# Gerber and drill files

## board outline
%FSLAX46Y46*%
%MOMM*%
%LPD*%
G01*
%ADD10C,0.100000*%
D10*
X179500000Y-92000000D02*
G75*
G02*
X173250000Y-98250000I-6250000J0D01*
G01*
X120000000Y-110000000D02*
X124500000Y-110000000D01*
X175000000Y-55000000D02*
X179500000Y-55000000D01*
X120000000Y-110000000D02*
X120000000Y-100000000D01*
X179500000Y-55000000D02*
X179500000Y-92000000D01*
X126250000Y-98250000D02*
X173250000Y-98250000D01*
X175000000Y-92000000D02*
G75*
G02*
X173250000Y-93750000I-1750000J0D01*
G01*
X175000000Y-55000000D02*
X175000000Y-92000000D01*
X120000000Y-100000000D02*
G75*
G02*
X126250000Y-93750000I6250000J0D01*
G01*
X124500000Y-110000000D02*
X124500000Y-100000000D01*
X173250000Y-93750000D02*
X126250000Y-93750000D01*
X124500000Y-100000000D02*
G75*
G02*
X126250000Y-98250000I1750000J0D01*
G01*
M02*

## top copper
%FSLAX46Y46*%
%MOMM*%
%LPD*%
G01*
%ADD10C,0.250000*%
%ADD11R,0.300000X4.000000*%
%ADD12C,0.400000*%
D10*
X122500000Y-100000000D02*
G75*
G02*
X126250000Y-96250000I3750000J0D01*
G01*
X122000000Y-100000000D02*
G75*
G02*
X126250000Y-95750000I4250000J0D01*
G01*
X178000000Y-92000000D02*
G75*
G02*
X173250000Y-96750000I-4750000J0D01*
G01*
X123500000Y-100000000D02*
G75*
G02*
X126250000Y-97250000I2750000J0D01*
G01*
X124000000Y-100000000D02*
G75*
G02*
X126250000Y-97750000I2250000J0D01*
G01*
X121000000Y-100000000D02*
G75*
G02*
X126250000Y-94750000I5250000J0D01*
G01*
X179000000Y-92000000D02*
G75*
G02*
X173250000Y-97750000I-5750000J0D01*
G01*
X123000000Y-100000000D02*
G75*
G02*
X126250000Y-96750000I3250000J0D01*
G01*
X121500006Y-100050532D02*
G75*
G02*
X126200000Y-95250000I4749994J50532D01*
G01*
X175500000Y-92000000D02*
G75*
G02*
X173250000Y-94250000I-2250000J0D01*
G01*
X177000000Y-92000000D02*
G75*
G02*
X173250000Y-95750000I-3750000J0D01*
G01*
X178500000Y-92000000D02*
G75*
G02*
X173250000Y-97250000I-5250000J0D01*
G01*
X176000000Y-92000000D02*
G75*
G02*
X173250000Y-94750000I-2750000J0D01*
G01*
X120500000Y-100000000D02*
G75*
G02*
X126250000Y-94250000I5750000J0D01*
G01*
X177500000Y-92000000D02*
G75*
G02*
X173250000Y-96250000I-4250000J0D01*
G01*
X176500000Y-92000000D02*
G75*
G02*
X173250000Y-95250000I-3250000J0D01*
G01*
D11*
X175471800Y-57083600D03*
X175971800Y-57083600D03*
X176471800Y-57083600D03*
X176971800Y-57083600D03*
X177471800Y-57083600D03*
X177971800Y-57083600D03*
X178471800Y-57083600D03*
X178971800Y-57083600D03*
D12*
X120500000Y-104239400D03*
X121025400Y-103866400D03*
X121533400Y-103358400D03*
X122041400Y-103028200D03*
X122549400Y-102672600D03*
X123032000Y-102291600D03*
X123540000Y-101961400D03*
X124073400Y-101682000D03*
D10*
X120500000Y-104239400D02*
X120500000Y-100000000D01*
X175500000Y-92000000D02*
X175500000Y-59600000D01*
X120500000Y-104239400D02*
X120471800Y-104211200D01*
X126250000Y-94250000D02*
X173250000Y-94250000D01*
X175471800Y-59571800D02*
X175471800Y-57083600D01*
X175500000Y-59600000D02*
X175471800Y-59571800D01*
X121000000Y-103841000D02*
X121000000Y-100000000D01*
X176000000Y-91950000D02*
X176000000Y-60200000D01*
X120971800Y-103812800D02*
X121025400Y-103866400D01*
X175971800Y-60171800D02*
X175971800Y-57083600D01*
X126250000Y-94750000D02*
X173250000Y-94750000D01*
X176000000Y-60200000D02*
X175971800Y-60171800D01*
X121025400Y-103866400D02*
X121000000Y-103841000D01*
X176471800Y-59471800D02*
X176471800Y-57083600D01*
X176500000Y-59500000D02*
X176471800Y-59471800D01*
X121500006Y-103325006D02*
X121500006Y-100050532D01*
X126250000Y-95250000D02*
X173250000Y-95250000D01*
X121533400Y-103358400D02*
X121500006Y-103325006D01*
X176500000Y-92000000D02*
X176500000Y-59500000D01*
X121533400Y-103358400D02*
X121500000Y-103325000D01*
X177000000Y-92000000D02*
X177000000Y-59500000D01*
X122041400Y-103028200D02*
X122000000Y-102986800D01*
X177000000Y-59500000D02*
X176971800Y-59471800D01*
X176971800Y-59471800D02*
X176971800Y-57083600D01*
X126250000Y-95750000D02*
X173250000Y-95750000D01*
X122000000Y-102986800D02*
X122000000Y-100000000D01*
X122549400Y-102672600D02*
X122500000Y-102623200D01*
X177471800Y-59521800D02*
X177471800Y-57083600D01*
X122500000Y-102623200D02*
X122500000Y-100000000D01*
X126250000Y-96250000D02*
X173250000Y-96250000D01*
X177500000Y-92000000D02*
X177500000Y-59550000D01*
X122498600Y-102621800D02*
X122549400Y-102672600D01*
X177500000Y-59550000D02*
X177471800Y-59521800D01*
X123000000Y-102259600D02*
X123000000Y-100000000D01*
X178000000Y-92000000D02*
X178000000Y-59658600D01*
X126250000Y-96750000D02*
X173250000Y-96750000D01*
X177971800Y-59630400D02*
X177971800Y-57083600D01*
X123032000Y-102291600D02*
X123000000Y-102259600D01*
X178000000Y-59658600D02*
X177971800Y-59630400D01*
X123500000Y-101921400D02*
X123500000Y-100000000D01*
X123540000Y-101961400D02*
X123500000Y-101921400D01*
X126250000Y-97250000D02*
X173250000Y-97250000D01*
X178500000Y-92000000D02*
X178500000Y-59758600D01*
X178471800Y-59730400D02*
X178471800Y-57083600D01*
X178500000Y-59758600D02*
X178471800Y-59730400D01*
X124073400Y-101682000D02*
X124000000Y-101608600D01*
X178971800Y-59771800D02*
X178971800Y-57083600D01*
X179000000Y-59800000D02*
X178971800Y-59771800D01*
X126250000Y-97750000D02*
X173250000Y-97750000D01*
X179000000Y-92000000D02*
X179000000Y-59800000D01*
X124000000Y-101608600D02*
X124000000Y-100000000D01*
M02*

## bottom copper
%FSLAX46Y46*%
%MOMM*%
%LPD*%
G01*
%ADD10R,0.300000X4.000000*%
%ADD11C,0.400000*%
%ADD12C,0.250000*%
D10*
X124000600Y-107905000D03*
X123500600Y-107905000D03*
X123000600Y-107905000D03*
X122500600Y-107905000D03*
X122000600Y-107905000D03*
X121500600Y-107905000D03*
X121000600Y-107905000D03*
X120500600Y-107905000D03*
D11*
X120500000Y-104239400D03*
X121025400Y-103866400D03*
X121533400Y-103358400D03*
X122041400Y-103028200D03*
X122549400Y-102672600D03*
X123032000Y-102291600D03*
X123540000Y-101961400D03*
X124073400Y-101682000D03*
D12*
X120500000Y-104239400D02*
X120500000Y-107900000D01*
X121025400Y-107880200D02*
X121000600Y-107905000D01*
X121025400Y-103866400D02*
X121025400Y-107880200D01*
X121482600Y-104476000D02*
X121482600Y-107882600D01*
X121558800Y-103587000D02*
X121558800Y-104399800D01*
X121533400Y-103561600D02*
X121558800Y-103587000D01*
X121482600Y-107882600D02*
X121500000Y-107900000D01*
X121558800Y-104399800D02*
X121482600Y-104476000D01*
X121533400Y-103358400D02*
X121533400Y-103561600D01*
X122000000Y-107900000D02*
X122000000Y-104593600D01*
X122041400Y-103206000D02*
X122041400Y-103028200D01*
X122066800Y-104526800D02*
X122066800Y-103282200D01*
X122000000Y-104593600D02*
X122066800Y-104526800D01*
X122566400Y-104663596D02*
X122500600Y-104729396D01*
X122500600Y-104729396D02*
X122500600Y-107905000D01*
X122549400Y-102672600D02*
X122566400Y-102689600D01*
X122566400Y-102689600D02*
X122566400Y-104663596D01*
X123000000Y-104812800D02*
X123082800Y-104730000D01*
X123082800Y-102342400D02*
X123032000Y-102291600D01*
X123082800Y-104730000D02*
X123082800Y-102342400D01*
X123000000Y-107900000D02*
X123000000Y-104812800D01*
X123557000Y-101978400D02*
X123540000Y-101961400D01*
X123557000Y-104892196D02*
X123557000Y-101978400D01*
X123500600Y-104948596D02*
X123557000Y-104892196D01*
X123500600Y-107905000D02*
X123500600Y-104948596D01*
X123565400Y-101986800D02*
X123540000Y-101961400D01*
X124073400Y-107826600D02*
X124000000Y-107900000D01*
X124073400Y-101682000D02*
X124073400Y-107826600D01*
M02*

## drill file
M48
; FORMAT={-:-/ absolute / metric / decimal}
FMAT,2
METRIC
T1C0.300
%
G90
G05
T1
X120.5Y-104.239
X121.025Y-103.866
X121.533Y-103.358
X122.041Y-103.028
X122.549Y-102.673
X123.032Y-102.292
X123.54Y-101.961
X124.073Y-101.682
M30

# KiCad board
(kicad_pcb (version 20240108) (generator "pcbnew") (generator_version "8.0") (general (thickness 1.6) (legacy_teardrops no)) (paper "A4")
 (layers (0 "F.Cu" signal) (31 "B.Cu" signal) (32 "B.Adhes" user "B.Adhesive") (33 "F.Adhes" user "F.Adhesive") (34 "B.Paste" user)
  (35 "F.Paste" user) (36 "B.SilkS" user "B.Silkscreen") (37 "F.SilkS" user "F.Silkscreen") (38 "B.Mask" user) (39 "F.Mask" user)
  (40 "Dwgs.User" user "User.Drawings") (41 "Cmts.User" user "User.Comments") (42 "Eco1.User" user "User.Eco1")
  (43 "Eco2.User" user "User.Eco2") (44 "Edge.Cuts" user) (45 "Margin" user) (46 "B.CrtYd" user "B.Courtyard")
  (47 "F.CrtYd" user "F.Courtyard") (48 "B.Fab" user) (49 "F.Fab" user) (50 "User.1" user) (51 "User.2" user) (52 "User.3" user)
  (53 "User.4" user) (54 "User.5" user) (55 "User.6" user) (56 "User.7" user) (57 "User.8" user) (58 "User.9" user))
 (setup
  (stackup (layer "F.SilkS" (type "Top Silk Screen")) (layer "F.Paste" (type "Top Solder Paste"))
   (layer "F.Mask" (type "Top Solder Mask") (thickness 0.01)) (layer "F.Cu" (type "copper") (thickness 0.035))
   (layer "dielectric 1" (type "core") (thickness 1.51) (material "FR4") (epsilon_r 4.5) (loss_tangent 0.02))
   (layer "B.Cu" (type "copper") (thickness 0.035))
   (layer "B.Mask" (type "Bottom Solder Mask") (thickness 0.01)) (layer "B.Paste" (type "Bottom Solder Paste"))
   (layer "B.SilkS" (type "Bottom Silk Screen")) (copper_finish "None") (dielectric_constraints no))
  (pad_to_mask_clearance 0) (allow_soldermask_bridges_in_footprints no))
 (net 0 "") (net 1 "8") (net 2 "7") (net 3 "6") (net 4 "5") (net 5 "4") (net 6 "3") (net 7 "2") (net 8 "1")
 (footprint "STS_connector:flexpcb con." (layer "F.Cu") (at 174.9718 59.0836)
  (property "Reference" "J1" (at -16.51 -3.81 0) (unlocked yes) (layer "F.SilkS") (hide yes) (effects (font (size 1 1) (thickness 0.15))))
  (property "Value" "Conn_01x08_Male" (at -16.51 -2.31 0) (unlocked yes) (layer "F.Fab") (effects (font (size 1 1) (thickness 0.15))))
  (pad "1" smd rect (at 0.5 -2) (size 0.3 4) (layers "F.Cu" "F.Paste" "F.Mask") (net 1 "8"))
  (pad "2" smd rect (at 1 -2) (size 0.3 4) (layers "F.Cu" "F.Paste" "F.Mask") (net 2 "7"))
  (pad "3" smd rect (at 1.5 -2) (size 0.3 4) (layers "F.Cu" "F.Paste" "F.Mask") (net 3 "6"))
  (pad "4" smd rect (at 2 -2) (size 0.3 4) (layers "F.Cu" "F.Paste" "F.Mask") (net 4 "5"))
  (pad "5" smd rect (at 2.5 -2) (size 0.3 4) (layers "F.Cu" "F.Paste" "F.Mask") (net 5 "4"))
  (pad "6" smd rect (at 3 -2) (size 0.3 4) (layers "F.Cu" "F.Paste" "F.Mask") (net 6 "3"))
  (pad "7" smd rect (at 3.5 -2) (size 0.3 4) (layers "F.Cu" "F.Paste" "F.Mask") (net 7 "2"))
  (pad "8" smd rect (at 4 -2) (size 0.3 4) (layers "F.Cu" "F.Paste" "F.Mask") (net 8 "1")))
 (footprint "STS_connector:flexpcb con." (layer "B.Cu") (at 124.5006 109.905 180)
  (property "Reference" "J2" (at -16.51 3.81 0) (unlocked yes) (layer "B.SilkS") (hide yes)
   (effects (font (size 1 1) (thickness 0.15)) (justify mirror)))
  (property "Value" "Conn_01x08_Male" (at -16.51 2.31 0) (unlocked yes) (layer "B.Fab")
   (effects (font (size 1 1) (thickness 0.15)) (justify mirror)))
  (pad "1" smd rect (at 0.5 2 180) (size 0.3 4) (layers "B.Cu" "B.Paste" "B.Mask") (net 8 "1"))
  (pad "2" smd rect (at 1 2 180) (size 0.3 4) (layers "B.Cu" "B.Paste" "B.Mask") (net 7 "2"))
  (pad "3" smd rect (at 1.5 2 180) (size 0.3 4) (layers "B.Cu" "B.Paste" "B.Mask") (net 6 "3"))
  (pad "4" smd rect (at 2 2 180) (size 0.3 4) (layers "B.Cu" "B.Paste" "B.Mask") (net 5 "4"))
  (pad "5" smd rect (at 2.5 2 180) (size 0.3 4) (layers "B.Cu" "B.Paste" "B.Mask") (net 4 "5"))
  (pad "6" smd rect (at 3 2 180) (size 0.3 4) (layers "B.Cu" "B.Paste" "B.Mask") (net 3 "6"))
  (pad "7" smd rect (at 3.5 2 180) (size 0.3 4) (layers "B.Cu" "B.Paste" "B.Mask") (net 2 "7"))
  (pad "8" smd rect (at 4 2 180) (size 0.3 4) (layers "B.Cu" "B.Paste" "B.Mask") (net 1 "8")))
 (gr_arc (start 122.5 100) (mid 123.59835 97.34835) (end 126.25 96.25) (stroke (width 0.25) (type default)) (layer "F.Cu") (net 5))
 (gr_arc (start 122 100) (mid 123.244796 96.994796) (end 126.25 95.75) (stroke (width 0.25) (type default)) (layer "F.Cu") (net 4))
 (gr_arc (start 178 92) (mid 176.608757 95.358757) (end 173.25 96.75) (stroke (width 0.25) (type default)) (layer "F.Cu") (net 6))
 (gr_arc (start 123.5 100) (mid 124.305456 98.055456) (end 126.25 97.25) (stroke (width 0.25) (type default)) (layer "F.Cu") (net 7))
 (gr_arc (start 124 100) (mid 124.65901 98.40901) (end 126.25 97.75) (stroke (width 0.25) (type default)) (layer "F.Cu") (net 8))
 (gr_arc (start 121 100) (mid 122.537689 96.287689) (end 126.25 94.75) (stroke (width 0.25) (type default)) (layer "F.Cu") (net 2))
 (gr_arc (start 179 92) (mid 177.315864 96.065864) (end 173.25 97.75) (stroke (width 0.25) (type default)) (layer "F.Cu") (net 8))
 (gr_arc (start 123 100) (mid 123.951903 97.701903) (end 126.25 96.75) (stroke (width 0.25) (type default)) (layer "F.Cu") (net 6))
 (gr_arc (start 121.500006 100.050532) (mid 122.855701 96.676788) (end 126.2 95.25) (stroke (width 0.25) (type default)) (layer "F.Cu")
  (net 3))
 (gr_arc (start 175.5 92) (mid 174.84099 93.59099) (end 173.25 94.25) (stroke (width 0.25) (type default)) (layer "F.Cu") (net 1))
 (gr_arc (start 177 92) (mid 175.90165 94.65165) (end 173.25 95.75) (stroke (width 0.25) (type default)) (layer "F.Cu") (net 4))
 (gr_arc (start 178.5 92) (mid 176.962311 95.712311) (end 173.25 97.25) (stroke (width 0.25) (type default)) (layer "F.Cu") (net 7))
 (gr_arc (start 176 92) (mid 175.194544 93.944544) (end 173.25 94.75) (stroke (width 0.25) (type default)) (layer "F.Cu") (net 2))
 (gr_arc (start 120.5 100) (mid 122.184136 95.934136) (end 126.25 94.25) (stroke (width 0.25) (type default)) (layer "F.Cu") (net 1))
 (gr_arc (start 177.5 92) (mid 176.255204 95.005204) (end 173.25 96.25) (stroke (width 0.25) (type default)) (layer "F.Cu") (net 5))
 (gr_arc (start 176.5 92) (mid 175.548097 94.298097) (end 173.25 95.25) (stroke (width 0.25) (type default)) (layer "F.Cu") (net 3))
 (gr_arc (start 179.5 92) (mid 177.669417 96.419417) (end 173.25 98.25) (stroke (width 0.1) (type default)) (layer "Edge.Cuts"))
 (gr_line (start 120 110) (end 124.5 110) (stroke (width 0.1) (type solid)) (layer "Edge.Cuts"))
 (gr_line (start 175 55) (end 179.5 55) (stroke (width 0.1) (type default)) (layer "Edge.Cuts"))
 (gr_line (start 120 110) (end 120 100) (stroke (width 0.1) (type default)) (layer "Edge.Cuts"))
 (gr_line (start 179.5 55) (end 179.5 92) (stroke (width 0.1) (type default)) (layer "Edge.Cuts"))
 (gr_line (start 126.25 98.25) (end 173.25 98.25) (stroke (width 0.1) (type default)) (layer "Edge.Cuts"))
 (gr_arc (start 175 92) (mid 174.487437 93.237437) (end 173.25 93.75) (stroke (width 0.1) (type default)) (layer "Edge.Cuts"))
 (gr_line (start 175 55) (end 175 92) (stroke (width 0.1) (type default)) (layer "Edge.Cuts"))
 (gr_arc (start 120 100) (mid 121.830583 95.580583) (end 126.25 93.75) (stroke (width 0.1) (type default)) (layer "Edge.Cuts"))
 (gr_line (start 124.5 110) (end 124.5 100) (stroke (width 0.1) (type default)) (layer "Edge.Cuts"))
 (gr_line (start 173.25 93.75) (end 126.25 93.75) (stroke (width 0.1) (type default)) (layer "Edge.Cuts"))
 (gr_arc (start 124.5 100) (mid 125.012563 98.762563) (end 126.25 98.25) (stroke (width 0.1) (type default)) (layer "Edge.Cuts"))
 (segment (start 120.5 104.2394) (end 120.5 100) (width 0.25) (layer "F.Cu") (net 1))
 (segment (start 175.5 92) (end 175.5 59.6) (width 0.25) (layer "F.Cu") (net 1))
 (segment (start 120.5 104.2394) (end 120.4718 104.2112) (width 0.25) (layer "F.Cu") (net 1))
 (segment (start 126.25 94.25) (end 173.25 94.25) (width 0.25) (layer "F.Cu") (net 1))
 (segment (start 175.4718 59.5718) (end 175.4718 57.0836) (width 0.25) (layer "F.Cu") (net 1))
 (segment (start 175.5 59.6) (end 175.4718 59.5718) (width 0.25) (layer "F.Cu") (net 1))
 (via (at 120.5 104.2394) (size 0.4) (drill 0.3) (layers "F.Cu" "B.Cu") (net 1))
 (segment (start 120.5 104.2394) (end 120.5 107.9) (width 0.25) (layer "B.Cu") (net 1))
 (segment (start 121 103.841) (end 121 100) (width 0.25) (layer "F.Cu") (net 2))
 (segment (start 176 91.95) (end 176 60.2) (width 0.25) (layer "F.Cu") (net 2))
 (segment (start 120.9718 103.8128) (end 121.0254 103.8664) (width 0.25) (layer "F.Cu") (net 2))
 (segment (start 175.9718 60.1718) (end 175.9718 57.0836) (width 0.25) (layer "F.Cu") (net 2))
 (segment (start 126.25 94.75) (end 173.25 94.75) (width 0.25) (layer "F.Cu") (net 2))
 (segment (start 176 60.2) (end 175.9718 60.1718) (width 0.25) (layer "F.Cu") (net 2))
 (segment (start 121.0254 103.8664) (end 121 103.841) (width 0.25) (layer "F.Cu") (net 2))
 (via (at 121.0254 103.8664) (size 0.4) (drill 0.3) (layers "F.Cu" "B.Cu") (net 2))
 (segment (start 121.0254 107.8802) (end 121.0006 107.905) (width 0.25) (layer "B.Cu") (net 2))
 (segment (start 121.0254 103.8664) (end 121.0254 107.8802) (width 0.25) (layer "B.Cu") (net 2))
 (segment (start 176.4718 59.4718) (end 176.4718 57.0836) (width 0.25) (layer "F.Cu") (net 3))
 (segment (start 176.5 59.5) (end 176.4718 59.4718) (width 0.25) (layer "F.Cu") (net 3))
 (segment (start 121.500006 103.325006) (end 121.500006 100.050532) (width 0.25) (layer "F.Cu") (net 3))
 (segment (start 126.25 95.25) (end 173.25 95.25) (width 0.25) (layer "F.Cu") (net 3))
 (segment (start 121.5334 103.3584) (end 121.500006 103.325006) (width 0.25) (layer "F.Cu") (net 3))
 (segment (start 176.5 92) (end 176.5 59.5) (width 0.25) (layer "F.Cu") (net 3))
 (segment (start 121.5334 103.3584) (end 121.5 103.325) (width 0.25) (layer "F.Cu") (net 3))
 (via (at 121.5334 103.3584) (size 0.4) (drill 0.3) (layers "F.Cu" "B.Cu") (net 3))
 (segment (start 121.4826 104.476) (end 121.4826 107.8826) (width 0.25) (layer "B.Cu") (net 3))
 (segment (start 121.5588 103.587) (end 121.5588 104.3998) (width 0.25) (layer "B.Cu") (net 3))
 (segment (start 121.5334 103.5616) (end 121.5588 103.587) (width 0.25) (layer "B.Cu") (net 3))
 (segment (start 121.4826 107.8826) (end 121.5 107.9) (width 0.25) (layer "B.Cu") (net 3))
 (segment (start 121.5588 104.3998) (end 121.4826 104.476) (width 0.25) (layer "B.Cu") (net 3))
 (segment (start 121.5334 103.3584) (end 121.5334 103.5616) (width 0.25) (layer "B.Cu") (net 3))
 (segment (start 177 92) (end 177 59.5) (width 0.25) (layer "F.Cu") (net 4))
 (segment (start 122.0414 103.0282) (end 122 102.9868) (width 0.25) (layer "F.Cu") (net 4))
 (segment (start 177 59.5) (end 176.9718 59.4718) (width 0.25) (layer "F.Cu") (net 4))
 (segment (start 176.9718 59.4718) (end 176.9718 57.0836) (width 0.25) (layer "F.Cu") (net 4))
 (segment (start 126.25 95.75) (end 173.25 95.75) (width 0.25) (layer "F.Cu") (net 4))
 (segment (start 122 102.9868) (end 122 100) (width 0.25) (layer "F.Cu") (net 4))
 (via (at 122.0414 103.0282) (size 0.4) (drill 0.3) (layers "F.Cu" "B.Cu") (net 4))
 (segment (start 122 107.9) (end 122 104.5936) (width 0.25) (layer "B.Cu") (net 4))
 (segment (start 122.0414 103.206) (end 122.0414 103.0282) (width 0.25) (layer "B.Cu") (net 4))
 (segment (start 122.0668 104.5268) (end 122.0668 103.2822) (width 0.25) (layer "B.Cu") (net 4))
 (segment (start 122 104.5936) (end 122.0668 104.5268) (width 0.25) (layer "B.Cu") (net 4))
 (segment (start 122.5494 102.6726) (end 122.5 102.6232) (width 0.25) (layer "F.Cu") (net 5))
 (segment (start 177.4718 59.5218) (end 177.4718 57.0836) (width 0.25) (layer "F.Cu") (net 5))
 (segment (start 122.5 102.6232) (end 122.5 100) (width 0.25) (layer "F.Cu") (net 5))
 (segment (start 126.25 96.25) (end 173.25 96.25) (width 0.25) (layer "F.Cu") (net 5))
 (segment (start 177.5 92) (end 177.5 59.55) (width 0.25) (layer "F.Cu") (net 5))
 (segment (start 122.4986 102.6218) (end 122.5494 102.6726) (width 0.25) (layer "F.Cu") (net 5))
 (segment (start 177.5 59.55) (end 177.4718 59.5218) (width 0.25) (layer "F.Cu") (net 5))
 (via (at 122.5494 102.6726) (size 0.4) (drill 0.3) (layers "F.Cu" "B.Cu") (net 5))
 (segment (start 122.5664 104.663596) (end 122.5006 104.729396) (width 0.25) (layer "B.Cu") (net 5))
 (segment (start 122.5006 104.729396) (end 122.5006 107.905) (width 0.25) (layer "B.Cu") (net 5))
 (segment (start 122.5494 102.6726) (end 122.5664 102.6896) (width 0.25) (layer "B.Cu") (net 5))
 (segment (start 122.5664 102.6896) (end 122.5664 104.663596) (width 0.25) (layer "B.Cu") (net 5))
 (segment (start 123 102.2596) (end 123 100) (width 0.25) (layer "F.Cu") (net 6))
 (segment (start 178 92) (end 178 59.6586) (width 0.25) (layer "F.Cu") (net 6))
 (segment (start 126.25 96.75) (end 173.25 96.75) (width 0.25) (layer "F.Cu") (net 6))
 (segment (start 177.9718 59.6304) (end 177.9718 57.0836) (width 0.25) (layer "F.Cu") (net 6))
 (segment (start 123.032 102.2916) (end 123 102.2596) (width 0.25) (layer "F.Cu") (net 6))
 (segment (start 178 59.6586) (end 177.9718 59.6304) (width 0.25) (layer "F.Cu") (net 6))
 (via (at 123.032 102.2916) (size 0.4) (drill 0.3) (layers "F.Cu" "B.Cu") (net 6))
 (segment (start 123 104.8128) (end 123.0828 104.73) (width 0.25) (layer "B.Cu") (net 6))
 (segment (start 123.0828 102.3424) (end 123.032 102.2916) (width 0.25) (layer "B.Cu") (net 6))
 (segment (start 123.0828 104.73) (end 123.0828 102.3424) (width 0.25) (layer "B.Cu") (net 6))
 (segment (start 123 107.9) (end 123 104.8128) (width 0.25) (layer "B.Cu") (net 6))
 (segment (start 123.5 101.9214) (end 123.5 100) (width 0.25) (layer "F.Cu") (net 7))
 (segment (start 123.54 101.9614) (end 123.5 101.9214) (width 0.25) (layer "F.Cu") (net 7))
 (segment (start 126.25 97.25) (end 173.25 97.25) (width 0.25) (layer "F.Cu") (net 7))
 (segment (start 178.5 92) (end 178.5 59.7586) (width 0.25) (layer "F.Cu") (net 7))
 (segment (start 178.4718 59.7304) (end 178.4718 57.0836) (width 0.25) (layer "F.Cu") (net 7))
 (segment (start 178.5 59.7586) (end 178.4718 59.7304) (width 0.25) (layer "F.Cu") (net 7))
 (via (at 123.54 101.9614) (size 0.4) (drill 0.3) (layers "F.Cu" "B.Cu") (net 7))
 (segment (start 123.557 101.9784) (end 123.54 101.9614) (width 0.25) (layer "B.Cu") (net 7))
 (segment (start 123.557 104.892196) (end 123.557 101.9784) (width 0.25) (layer "B.Cu") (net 7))
 (segment (start 123.5006 104.948596) (end 123.557 104.892196) (width 0.25) (layer "B.Cu") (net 7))
 (segment (start 123.5006 107.905) (end 123.5006 104.948596) (width 0.25) (layer "B.Cu") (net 7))
 (segment (start 123.5654 101.9868) (end 123.54 101.9614) (width 0.25) (layer "B.Cu") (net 7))
 (segment (start 124.0734 101.682) (end 124 101.6086) (width 0.25) (layer "F.Cu") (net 8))
 (segment (start 178.9718 59.7718) (end 178.9718 57.0836) (width 0.25) (layer "F.Cu") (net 8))
 (segment (start 179 59.8) (end 178.9718 59.7718) (width 0.25) (layer "F.Cu") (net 8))
 (segment (start 126.25 97.75) (end 173.25 97.75) (width 0.25) (layer "F.Cu") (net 8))
 (segment (start 179 92) (end 179 59.8) (width 0.25) (layer "F.Cu") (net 8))
 (segment (start 124 101.6086) (end 124 100) (width 0.25) (layer "F.Cu") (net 8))
 (via (at 124.0734 101.682) (size 0.4) (drill 0.3) (layers "F.Cu" "B.Cu") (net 8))
 (segment (start 124.0734 107.8266) (end 124 107.9) (width 0.25) (layer "B.Cu") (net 8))
 (segment (start 124.0734 101.682) (end 124.0734 107.8266) (width 0.25) (layer "B.Cu") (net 8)))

